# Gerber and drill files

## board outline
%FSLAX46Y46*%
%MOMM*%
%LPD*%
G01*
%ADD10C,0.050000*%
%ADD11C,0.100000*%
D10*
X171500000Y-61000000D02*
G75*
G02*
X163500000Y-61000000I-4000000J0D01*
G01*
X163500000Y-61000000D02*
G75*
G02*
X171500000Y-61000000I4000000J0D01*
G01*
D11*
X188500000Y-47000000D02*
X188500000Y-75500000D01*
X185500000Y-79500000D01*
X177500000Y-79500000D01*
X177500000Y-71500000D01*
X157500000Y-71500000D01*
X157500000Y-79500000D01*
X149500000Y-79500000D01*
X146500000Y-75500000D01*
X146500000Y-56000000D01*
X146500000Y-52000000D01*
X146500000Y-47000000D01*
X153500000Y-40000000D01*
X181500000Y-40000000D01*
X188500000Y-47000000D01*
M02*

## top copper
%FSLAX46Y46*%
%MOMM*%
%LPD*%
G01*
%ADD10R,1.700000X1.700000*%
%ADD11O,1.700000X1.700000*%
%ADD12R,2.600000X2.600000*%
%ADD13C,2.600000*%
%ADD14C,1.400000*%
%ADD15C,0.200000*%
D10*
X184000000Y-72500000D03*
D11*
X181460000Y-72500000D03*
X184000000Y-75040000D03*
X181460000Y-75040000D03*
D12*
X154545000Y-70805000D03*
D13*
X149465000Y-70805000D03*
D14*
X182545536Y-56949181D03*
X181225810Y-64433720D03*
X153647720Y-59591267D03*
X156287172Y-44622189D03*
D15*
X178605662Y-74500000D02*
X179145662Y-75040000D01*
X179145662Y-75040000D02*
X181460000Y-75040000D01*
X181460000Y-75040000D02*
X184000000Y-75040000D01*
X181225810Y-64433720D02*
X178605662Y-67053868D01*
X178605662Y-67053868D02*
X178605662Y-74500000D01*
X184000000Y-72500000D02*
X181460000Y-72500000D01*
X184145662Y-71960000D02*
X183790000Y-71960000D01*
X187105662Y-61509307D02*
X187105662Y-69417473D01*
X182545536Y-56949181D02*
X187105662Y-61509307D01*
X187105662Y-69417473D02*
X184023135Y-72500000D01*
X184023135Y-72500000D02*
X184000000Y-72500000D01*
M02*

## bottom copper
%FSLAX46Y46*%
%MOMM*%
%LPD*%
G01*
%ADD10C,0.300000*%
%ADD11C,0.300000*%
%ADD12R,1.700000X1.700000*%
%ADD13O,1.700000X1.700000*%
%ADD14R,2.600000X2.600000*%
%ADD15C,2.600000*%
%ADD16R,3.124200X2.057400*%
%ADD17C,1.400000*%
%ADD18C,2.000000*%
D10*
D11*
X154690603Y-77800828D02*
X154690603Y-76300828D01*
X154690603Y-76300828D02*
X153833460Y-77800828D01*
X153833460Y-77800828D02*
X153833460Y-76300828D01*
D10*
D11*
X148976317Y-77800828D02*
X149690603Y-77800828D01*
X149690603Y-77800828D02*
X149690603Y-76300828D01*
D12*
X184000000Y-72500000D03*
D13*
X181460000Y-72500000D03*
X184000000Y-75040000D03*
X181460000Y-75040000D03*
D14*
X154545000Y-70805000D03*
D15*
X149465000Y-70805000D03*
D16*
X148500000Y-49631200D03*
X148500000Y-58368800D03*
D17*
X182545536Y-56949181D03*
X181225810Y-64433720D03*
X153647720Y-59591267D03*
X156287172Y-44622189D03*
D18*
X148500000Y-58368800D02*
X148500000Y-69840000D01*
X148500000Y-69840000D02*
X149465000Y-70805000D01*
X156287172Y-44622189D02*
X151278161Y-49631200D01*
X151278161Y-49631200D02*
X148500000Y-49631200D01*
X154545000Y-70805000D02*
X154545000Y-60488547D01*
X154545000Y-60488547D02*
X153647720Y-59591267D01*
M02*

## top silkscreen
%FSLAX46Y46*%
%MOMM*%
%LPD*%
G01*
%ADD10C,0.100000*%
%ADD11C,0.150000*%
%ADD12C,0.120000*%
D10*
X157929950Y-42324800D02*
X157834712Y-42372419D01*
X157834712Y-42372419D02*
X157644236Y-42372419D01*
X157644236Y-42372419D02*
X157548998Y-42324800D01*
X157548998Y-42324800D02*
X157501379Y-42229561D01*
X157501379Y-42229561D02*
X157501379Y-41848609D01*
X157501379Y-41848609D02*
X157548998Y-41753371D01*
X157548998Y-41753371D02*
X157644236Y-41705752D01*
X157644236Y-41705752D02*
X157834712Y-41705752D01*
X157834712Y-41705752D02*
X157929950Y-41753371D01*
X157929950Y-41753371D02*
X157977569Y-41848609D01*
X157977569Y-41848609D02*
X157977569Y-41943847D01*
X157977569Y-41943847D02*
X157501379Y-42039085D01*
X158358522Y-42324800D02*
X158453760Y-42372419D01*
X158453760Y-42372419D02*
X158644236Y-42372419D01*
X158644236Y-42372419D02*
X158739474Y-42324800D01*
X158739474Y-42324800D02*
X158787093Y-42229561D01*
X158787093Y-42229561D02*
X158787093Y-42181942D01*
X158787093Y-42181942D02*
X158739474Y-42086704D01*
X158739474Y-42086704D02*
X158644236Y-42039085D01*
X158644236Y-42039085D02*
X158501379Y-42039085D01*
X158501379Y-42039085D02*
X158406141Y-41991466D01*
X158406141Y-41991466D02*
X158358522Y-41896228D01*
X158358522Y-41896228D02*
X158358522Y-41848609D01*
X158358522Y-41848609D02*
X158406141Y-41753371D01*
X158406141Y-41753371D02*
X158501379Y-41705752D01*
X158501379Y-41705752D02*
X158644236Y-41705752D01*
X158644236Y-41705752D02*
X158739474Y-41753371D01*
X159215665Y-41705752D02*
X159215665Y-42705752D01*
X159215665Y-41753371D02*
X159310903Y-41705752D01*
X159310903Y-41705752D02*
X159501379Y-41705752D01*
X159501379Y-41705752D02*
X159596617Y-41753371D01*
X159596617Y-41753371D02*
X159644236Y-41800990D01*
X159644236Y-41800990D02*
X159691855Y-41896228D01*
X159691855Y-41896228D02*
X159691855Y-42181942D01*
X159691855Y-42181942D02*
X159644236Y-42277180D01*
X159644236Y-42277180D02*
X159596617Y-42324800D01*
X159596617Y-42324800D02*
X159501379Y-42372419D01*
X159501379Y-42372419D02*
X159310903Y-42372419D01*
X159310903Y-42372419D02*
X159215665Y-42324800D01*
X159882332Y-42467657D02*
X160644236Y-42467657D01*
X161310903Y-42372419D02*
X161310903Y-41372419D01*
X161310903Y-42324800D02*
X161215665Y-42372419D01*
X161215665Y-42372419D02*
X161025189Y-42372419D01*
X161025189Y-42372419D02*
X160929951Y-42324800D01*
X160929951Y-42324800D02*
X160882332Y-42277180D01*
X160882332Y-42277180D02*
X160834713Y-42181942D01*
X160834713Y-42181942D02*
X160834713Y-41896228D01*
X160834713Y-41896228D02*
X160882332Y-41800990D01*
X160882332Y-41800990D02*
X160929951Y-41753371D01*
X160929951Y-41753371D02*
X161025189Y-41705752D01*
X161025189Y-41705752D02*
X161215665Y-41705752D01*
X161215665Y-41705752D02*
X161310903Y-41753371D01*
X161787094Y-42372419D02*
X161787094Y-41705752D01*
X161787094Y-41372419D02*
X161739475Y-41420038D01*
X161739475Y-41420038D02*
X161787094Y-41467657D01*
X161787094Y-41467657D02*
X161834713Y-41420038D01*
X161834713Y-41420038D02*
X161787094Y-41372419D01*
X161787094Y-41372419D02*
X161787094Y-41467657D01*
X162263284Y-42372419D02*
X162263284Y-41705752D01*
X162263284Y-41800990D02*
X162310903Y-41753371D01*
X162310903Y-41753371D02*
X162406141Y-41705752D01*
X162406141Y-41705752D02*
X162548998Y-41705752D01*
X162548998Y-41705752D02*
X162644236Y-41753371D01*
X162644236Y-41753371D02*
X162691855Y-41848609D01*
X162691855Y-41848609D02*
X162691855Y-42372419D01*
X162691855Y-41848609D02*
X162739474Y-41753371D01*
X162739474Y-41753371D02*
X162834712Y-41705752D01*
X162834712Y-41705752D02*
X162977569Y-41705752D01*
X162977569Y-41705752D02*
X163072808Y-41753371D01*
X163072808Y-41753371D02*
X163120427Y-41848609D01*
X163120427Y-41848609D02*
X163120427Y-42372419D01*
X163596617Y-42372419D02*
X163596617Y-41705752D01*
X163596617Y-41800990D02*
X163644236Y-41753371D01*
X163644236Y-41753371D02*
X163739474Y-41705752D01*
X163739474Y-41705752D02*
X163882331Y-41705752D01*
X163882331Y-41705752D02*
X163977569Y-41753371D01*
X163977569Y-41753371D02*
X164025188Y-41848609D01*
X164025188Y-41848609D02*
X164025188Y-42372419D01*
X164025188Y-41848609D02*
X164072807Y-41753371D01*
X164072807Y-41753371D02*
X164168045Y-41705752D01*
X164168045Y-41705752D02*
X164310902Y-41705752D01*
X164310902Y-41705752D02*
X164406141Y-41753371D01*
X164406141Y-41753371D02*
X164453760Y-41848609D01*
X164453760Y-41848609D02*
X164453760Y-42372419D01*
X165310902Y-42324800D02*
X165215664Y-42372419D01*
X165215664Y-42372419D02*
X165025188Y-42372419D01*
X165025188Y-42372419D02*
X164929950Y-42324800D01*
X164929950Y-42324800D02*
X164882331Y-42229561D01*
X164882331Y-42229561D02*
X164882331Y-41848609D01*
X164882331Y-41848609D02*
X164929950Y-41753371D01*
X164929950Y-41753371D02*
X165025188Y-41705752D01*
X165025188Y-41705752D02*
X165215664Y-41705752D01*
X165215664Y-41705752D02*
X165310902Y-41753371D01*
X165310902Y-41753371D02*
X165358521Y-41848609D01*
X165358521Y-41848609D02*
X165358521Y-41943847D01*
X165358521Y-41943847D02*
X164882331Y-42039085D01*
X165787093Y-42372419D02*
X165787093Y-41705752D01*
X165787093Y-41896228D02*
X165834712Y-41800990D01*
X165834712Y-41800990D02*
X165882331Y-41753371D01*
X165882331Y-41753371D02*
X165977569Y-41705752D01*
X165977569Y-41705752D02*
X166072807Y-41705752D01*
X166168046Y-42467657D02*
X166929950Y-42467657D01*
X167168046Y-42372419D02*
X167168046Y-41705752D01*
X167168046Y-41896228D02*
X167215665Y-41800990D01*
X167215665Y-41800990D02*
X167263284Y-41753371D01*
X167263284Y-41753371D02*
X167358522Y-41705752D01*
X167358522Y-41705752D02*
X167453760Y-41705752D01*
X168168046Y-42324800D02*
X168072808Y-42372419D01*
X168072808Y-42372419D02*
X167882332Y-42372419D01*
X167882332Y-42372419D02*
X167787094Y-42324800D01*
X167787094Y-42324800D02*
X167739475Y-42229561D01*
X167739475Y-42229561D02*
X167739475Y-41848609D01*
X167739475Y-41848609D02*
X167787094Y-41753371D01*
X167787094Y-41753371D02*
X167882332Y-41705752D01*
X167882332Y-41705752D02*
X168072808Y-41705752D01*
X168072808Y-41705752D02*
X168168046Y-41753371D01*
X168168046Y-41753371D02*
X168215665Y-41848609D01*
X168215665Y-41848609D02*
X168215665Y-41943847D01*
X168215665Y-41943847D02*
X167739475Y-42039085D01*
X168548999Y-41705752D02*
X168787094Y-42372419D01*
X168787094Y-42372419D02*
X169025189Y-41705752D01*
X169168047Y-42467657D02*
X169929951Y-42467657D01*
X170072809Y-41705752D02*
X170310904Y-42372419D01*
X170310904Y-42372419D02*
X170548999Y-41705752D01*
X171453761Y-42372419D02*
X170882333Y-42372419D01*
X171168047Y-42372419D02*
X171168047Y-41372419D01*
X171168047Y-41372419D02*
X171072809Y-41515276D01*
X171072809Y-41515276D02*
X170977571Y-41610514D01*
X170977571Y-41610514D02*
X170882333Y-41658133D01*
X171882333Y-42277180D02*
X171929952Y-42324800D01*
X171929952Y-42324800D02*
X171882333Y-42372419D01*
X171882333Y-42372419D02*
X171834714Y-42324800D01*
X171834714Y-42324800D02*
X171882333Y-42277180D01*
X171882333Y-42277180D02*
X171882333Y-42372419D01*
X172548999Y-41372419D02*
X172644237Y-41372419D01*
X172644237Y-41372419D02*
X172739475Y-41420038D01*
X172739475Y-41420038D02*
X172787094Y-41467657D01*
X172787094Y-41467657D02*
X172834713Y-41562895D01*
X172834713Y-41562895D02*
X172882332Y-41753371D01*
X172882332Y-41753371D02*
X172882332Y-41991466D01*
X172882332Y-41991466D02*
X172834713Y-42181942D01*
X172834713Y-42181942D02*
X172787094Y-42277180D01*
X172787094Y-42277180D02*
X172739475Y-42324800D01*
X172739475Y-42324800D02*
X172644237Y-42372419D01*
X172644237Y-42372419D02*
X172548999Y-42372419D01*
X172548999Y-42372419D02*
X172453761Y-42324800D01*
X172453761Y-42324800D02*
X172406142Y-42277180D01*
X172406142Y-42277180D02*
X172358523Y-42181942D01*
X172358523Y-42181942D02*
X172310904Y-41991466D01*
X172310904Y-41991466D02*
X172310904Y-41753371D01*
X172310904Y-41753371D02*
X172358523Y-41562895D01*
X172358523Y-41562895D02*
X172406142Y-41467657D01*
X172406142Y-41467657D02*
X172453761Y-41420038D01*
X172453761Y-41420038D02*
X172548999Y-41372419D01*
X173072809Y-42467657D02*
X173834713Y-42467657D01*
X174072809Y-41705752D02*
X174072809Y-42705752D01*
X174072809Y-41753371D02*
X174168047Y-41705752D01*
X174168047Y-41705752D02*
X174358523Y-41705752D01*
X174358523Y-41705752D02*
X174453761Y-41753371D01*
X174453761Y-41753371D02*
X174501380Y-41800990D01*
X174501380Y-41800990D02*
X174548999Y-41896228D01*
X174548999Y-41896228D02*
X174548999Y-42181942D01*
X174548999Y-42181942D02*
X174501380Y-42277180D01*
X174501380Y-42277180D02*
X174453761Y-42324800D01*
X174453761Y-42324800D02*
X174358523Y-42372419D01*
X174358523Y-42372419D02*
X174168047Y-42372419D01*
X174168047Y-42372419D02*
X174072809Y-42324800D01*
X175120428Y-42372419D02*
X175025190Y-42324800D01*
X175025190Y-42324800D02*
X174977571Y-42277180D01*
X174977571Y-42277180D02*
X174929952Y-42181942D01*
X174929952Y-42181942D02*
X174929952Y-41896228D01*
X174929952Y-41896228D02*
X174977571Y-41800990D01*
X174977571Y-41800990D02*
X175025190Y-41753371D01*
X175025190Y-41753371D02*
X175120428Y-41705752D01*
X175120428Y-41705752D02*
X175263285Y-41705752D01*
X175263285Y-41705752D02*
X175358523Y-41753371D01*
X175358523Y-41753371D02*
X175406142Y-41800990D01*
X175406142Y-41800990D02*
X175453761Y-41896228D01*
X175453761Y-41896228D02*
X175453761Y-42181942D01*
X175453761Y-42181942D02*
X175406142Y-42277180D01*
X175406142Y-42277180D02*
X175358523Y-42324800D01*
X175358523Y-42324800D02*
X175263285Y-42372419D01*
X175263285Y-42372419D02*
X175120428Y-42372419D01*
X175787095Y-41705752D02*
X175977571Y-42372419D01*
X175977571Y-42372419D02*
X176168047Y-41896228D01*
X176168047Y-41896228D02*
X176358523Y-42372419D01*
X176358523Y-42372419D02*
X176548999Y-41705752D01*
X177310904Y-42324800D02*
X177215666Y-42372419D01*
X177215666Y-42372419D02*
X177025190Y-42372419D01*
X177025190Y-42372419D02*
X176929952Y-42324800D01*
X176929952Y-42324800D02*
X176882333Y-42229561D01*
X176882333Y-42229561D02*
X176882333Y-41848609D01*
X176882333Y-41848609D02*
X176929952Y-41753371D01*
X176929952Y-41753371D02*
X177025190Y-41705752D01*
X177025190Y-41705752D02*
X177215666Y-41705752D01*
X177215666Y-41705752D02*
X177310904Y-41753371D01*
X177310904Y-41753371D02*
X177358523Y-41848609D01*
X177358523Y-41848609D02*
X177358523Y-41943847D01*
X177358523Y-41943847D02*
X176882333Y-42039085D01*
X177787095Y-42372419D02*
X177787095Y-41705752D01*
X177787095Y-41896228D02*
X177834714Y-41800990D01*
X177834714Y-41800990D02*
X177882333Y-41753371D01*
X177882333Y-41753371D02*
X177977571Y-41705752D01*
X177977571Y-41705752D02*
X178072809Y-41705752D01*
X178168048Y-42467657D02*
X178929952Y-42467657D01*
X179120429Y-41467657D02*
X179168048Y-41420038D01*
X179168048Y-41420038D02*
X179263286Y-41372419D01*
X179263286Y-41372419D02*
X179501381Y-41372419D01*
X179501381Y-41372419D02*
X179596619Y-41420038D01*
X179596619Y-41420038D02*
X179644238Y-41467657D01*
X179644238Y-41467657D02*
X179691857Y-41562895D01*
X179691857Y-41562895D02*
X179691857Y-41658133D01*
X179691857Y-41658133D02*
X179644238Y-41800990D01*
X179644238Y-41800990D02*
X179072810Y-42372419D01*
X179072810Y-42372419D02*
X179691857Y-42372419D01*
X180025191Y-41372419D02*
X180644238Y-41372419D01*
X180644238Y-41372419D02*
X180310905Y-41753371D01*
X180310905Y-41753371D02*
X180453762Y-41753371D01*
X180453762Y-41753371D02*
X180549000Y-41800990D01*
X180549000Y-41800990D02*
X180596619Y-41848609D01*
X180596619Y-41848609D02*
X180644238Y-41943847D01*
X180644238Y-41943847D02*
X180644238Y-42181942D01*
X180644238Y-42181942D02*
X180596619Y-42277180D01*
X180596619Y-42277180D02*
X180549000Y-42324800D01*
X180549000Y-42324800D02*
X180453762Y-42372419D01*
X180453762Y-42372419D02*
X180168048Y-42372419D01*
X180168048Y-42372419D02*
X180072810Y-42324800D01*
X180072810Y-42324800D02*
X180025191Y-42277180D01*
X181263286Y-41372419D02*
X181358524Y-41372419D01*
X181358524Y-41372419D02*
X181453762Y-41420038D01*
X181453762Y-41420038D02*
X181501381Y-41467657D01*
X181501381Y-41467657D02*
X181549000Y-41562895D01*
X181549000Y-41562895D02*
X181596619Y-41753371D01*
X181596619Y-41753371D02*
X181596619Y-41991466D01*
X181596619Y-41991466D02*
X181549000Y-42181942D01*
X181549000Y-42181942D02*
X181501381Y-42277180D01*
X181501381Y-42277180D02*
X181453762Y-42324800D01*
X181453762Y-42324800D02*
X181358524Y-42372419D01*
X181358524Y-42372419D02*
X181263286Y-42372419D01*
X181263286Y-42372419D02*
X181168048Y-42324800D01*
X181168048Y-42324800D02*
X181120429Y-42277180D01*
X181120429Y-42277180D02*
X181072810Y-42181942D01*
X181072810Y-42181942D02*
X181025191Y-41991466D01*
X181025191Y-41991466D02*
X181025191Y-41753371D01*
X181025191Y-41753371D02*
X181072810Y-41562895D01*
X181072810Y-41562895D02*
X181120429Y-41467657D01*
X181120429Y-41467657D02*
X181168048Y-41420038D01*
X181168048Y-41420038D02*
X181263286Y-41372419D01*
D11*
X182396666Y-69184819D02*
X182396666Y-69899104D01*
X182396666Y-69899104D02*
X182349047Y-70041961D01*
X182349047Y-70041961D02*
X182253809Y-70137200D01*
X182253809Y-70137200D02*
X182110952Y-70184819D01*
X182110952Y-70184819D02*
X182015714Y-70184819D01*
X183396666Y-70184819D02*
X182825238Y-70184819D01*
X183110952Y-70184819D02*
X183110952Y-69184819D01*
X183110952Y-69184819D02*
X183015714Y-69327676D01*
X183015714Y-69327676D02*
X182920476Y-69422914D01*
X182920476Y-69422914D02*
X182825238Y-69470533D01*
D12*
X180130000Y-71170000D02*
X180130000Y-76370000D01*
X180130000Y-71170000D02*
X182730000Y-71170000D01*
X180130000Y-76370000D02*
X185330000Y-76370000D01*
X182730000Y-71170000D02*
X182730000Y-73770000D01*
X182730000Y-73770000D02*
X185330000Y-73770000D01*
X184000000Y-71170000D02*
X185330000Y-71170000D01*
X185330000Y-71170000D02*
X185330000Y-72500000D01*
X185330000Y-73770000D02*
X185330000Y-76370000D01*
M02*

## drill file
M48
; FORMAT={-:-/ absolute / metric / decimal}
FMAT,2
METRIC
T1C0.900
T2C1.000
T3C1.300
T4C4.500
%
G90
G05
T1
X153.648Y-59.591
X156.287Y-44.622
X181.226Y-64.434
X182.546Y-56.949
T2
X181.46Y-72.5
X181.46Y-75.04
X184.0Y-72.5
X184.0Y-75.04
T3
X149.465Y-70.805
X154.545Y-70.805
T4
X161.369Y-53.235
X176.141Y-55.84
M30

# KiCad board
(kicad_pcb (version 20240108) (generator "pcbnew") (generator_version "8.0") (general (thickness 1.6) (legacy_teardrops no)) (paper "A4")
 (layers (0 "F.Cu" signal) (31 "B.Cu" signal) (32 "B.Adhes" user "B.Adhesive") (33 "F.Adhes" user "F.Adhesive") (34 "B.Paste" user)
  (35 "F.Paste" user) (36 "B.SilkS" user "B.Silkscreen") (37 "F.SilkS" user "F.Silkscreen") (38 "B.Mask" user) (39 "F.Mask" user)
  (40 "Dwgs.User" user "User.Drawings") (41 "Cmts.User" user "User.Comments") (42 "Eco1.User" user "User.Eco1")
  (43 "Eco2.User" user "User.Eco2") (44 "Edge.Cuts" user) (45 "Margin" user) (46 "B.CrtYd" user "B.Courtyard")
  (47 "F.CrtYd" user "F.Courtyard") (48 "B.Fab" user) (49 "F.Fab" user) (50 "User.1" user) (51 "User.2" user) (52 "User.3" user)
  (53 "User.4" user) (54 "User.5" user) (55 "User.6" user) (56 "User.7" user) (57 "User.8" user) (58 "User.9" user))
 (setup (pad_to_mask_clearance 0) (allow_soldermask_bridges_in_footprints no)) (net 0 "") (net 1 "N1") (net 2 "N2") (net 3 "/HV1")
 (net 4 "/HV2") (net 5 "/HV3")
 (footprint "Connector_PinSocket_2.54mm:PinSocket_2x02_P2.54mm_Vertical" (layer "F.Cu") (at 184 72.5)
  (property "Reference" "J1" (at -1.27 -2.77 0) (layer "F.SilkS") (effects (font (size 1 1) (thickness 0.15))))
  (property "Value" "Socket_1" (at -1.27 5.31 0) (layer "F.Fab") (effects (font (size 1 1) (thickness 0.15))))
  (fp_line (start -3.87 -1.33) (end -3.87 3.87) (stroke (width 0.12) (type solid)) (layer "F.SilkS"))
  (fp_line (start -3.87 -1.33) (end -1.27 -1.33) (stroke (width 0.12) (type solid)) (layer "F.SilkS"))
  (fp_line (start -3.87 3.87) (end 1.33 3.87) (stroke (width 0.12) (type solid)) (layer "F.SilkS"))
  (fp_line (start -1.27 -1.33) (end -1.27 1.27) (stroke (width 0.12) (type solid)) (layer "F.SilkS"))
  (fp_line (start -1.27 1.27) (end 1.33 1.27) (stroke (width 0.12) (type solid)) (layer "F.SilkS"))
  (fp_line (start 0 -1.33) (end 1.33 -1.33) (stroke (width 0.12) (type solid)) (layer "F.SilkS"))
  (fp_line (start 1.33 -1.33) (end 1.33 0) (stroke (width 0.12) (type solid)) (layer "F.SilkS"))
  (fp_line (start 1.33 1.27) (end 1.33 3.87) (stroke (width 0.12) (type solid)) (layer "F.SilkS"))
  (pad "1" thru_hole rect (at 0 0) (size 1.7 1.7) (drill 1) (layers "*.Cu" "*.Mask") (remove_unused_layers no) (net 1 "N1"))
  (pad "2" thru_hole oval (at -2.54 0) (size 1.7 1.7) (drill 1) (layers "*.Cu" "*.Mask") (remove_unused_layers no) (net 1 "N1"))
  (pad "3" thru_hole oval (at 0 2.54) (size 1.7 1.7) (drill 1) (layers "*.Cu" "*.Mask") (remove_unused_layers no) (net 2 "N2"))
  (pad "4" thru_hole oval (at -2.54 2.54) (size 1.7 1.7) (drill 1) (layers "*.Cu" "*.Mask") (remove_unused_layers no) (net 2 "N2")))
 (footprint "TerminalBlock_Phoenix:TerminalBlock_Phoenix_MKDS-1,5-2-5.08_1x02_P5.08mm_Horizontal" (layer "B.Cu") (at 154.545 70.805 180)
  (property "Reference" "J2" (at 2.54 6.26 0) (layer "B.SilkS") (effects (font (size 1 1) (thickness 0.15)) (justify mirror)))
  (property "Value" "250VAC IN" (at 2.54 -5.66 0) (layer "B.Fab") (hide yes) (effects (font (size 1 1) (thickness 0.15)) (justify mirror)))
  (pad "1" thru_hole rect (at 0 0 180) (size 2.6 2.6) (drill 1.3) (layers "*.Cu" "*.Mask") (remove_unused_layers no) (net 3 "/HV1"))
  (pad "2" thru_hole circle (at 5.08 0 180) (size 2.6 2.6) (drill 1.3) (layers "*.Cu" "*.Mask") (remove_unused_layers no) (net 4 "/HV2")))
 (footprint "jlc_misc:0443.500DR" (layer "B.Cu") (at 148.5 54 -90)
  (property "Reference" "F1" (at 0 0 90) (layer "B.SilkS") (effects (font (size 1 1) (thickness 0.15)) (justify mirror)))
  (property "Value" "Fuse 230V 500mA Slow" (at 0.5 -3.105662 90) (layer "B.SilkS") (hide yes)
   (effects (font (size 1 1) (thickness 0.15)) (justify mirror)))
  (pad "1" smd rect (at -4.3688 0 270) (size 2.0574 3.1242) (layers "B.Cu" "B.Paste" "B.Mask") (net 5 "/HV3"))
  (pad "2" smd rect (at 4.3688 0 270) (size 2.0574 3.1242) (layers "B.Cu" "B.Paste" "B.Mask") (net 4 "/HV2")))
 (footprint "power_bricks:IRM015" (layer "B.Cu") (at 182.545536 56.949181 170)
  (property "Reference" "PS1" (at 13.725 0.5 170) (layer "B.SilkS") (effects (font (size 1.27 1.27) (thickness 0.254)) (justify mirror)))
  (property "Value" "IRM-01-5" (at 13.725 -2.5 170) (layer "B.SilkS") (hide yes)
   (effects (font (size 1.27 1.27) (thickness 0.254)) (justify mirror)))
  (pad "" np_thru_hole circle (at 6.5 -0.02 170) (size 4.5 4.5) (drill 4.5) (layers "*.Cu" "*.Mask"))
  (pad "" np_thru_hole circle (at 21.5 -0.02 170) (size 4.5 4.5) (drill 4.5) (layers "*.Cu" "*.Mask"))
  (pad "1" thru_hole circle (at 0 0 170) (size 1.4 1.4) (drill 0.9) (layers "*.Cu" "*.Mask") (remove_unused_layers no) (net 1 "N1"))
  (pad "2" thru_hole circle (at 0 -7.6 170) (size 1.4 1.4) (drill 0.9) (layers "*.Cu" "*.Mask") (remove_unused_layers no) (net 2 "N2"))
  (pad "3" thru_hole circle (at 28 -7.62 170) (size 1.4 1.4) (drill 0.9) (layers "*.Cu" "*.Mask") (remove_unused_layers no) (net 3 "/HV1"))
  (pad "4" thru_hole circle (at 28 7.58 170) (size 1.4 1.4) (drill 0.9) (layers "*.Cu" "*.Mask") (remove_unused_layers no) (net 5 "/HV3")))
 (gr_circle (center 167.5 61) (end 171.5 61) (stroke (width 0.05) (type default)) (fill none) (layer "Edge.Cuts"))
 (gr_poly
  (pts (xy 188.5 47) (xy 188.5 75.5) (xy 185.5 79.5) (xy 177.5 79.5) (xy 177.5 71.5) (xy 157.5 71.5) (xy 157.5 79.5) (xy 149.5 79.5)
   (xy 146.5 75.5) (xy 146.5 56) (xy 146.5 52) (xy 146.5 47) (xy 153.5 40) (xy 181.5 40))
  (stroke (width 0.1) (type solid)) (fill none) (layer "Edge.Cuts"))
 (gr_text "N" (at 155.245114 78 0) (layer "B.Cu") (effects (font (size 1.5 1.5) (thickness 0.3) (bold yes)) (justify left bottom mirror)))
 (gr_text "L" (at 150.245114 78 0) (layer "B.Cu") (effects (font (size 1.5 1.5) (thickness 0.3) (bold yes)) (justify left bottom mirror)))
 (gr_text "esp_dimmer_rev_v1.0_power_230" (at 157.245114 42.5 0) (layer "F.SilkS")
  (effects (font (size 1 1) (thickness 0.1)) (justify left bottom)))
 (segment (start 178.605662 74.5) (end 179.145662 75.04) (width 0.2) (layer "F.Cu") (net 2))
 (segment (start 179.145662 75.04) (end 181.46 75.04) (width 0.2) (layer "F.Cu") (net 2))
 (segment (start 181.46 75.04) (end 184 75.04) (width 0.2) (layer "F.Cu") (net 2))
 (segment (start 181.22581 64.43372) (end 178.605662 67.053868) (width 0.2) (layer "F.Cu") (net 2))
 (segment (start 178.605662 67.053868) (end 178.605662 74.5) (width 0.2) (layer "F.Cu") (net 2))
 (segment (start 184 72.5) (end 181.46 72.5) (width 0.2) (layer "F.Cu") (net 1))
 (segment (start 184.145662 71.96) (end 183.79 71.96) (width 0.2) (layer "F.Cu") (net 1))
 (segment (start 187.105662 61.509307) (end 187.105662 69.417473) (width 0.2) (layer "F.Cu") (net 1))
 (segment (start 182.545536 56.949181) (end 187.105662 61.509307) (width 0.2) (layer "F.Cu") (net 1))
 (segment (start 187.105662 69.417473) (end 184.023135 72.5) (width 0.2) (layer "F.Cu") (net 1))
 (segment (start 184.023135 72.5) (end 184 72.5) (width 0.2) (layer "F.Cu") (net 1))
 (segment (start 148.5 58.3688) (end 148.5 69.84) (width 2) (layer "B.Cu") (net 4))
 (segment (start 148.5 69.84) (end 149.465 70.805) (width 2) (layer "B.Cu") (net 4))
 (segment (start 156.287172 44.622189) (end 151.278161 49.6312) (width 2) (layer "B.Cu") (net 5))
 (segment (start 151.278161 49.6312) (end 148.5 49.6312) (width 2) (layer "B.Cu") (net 5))
 (segment (start 154.545 70.805) (end 154.545 60.488547) (width 2) (layer "B.Cu") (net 3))
 (segment (start 154.545 60.488547) (end 153.64772 59.591267) (width 2) (layer "B.Cu") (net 3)))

